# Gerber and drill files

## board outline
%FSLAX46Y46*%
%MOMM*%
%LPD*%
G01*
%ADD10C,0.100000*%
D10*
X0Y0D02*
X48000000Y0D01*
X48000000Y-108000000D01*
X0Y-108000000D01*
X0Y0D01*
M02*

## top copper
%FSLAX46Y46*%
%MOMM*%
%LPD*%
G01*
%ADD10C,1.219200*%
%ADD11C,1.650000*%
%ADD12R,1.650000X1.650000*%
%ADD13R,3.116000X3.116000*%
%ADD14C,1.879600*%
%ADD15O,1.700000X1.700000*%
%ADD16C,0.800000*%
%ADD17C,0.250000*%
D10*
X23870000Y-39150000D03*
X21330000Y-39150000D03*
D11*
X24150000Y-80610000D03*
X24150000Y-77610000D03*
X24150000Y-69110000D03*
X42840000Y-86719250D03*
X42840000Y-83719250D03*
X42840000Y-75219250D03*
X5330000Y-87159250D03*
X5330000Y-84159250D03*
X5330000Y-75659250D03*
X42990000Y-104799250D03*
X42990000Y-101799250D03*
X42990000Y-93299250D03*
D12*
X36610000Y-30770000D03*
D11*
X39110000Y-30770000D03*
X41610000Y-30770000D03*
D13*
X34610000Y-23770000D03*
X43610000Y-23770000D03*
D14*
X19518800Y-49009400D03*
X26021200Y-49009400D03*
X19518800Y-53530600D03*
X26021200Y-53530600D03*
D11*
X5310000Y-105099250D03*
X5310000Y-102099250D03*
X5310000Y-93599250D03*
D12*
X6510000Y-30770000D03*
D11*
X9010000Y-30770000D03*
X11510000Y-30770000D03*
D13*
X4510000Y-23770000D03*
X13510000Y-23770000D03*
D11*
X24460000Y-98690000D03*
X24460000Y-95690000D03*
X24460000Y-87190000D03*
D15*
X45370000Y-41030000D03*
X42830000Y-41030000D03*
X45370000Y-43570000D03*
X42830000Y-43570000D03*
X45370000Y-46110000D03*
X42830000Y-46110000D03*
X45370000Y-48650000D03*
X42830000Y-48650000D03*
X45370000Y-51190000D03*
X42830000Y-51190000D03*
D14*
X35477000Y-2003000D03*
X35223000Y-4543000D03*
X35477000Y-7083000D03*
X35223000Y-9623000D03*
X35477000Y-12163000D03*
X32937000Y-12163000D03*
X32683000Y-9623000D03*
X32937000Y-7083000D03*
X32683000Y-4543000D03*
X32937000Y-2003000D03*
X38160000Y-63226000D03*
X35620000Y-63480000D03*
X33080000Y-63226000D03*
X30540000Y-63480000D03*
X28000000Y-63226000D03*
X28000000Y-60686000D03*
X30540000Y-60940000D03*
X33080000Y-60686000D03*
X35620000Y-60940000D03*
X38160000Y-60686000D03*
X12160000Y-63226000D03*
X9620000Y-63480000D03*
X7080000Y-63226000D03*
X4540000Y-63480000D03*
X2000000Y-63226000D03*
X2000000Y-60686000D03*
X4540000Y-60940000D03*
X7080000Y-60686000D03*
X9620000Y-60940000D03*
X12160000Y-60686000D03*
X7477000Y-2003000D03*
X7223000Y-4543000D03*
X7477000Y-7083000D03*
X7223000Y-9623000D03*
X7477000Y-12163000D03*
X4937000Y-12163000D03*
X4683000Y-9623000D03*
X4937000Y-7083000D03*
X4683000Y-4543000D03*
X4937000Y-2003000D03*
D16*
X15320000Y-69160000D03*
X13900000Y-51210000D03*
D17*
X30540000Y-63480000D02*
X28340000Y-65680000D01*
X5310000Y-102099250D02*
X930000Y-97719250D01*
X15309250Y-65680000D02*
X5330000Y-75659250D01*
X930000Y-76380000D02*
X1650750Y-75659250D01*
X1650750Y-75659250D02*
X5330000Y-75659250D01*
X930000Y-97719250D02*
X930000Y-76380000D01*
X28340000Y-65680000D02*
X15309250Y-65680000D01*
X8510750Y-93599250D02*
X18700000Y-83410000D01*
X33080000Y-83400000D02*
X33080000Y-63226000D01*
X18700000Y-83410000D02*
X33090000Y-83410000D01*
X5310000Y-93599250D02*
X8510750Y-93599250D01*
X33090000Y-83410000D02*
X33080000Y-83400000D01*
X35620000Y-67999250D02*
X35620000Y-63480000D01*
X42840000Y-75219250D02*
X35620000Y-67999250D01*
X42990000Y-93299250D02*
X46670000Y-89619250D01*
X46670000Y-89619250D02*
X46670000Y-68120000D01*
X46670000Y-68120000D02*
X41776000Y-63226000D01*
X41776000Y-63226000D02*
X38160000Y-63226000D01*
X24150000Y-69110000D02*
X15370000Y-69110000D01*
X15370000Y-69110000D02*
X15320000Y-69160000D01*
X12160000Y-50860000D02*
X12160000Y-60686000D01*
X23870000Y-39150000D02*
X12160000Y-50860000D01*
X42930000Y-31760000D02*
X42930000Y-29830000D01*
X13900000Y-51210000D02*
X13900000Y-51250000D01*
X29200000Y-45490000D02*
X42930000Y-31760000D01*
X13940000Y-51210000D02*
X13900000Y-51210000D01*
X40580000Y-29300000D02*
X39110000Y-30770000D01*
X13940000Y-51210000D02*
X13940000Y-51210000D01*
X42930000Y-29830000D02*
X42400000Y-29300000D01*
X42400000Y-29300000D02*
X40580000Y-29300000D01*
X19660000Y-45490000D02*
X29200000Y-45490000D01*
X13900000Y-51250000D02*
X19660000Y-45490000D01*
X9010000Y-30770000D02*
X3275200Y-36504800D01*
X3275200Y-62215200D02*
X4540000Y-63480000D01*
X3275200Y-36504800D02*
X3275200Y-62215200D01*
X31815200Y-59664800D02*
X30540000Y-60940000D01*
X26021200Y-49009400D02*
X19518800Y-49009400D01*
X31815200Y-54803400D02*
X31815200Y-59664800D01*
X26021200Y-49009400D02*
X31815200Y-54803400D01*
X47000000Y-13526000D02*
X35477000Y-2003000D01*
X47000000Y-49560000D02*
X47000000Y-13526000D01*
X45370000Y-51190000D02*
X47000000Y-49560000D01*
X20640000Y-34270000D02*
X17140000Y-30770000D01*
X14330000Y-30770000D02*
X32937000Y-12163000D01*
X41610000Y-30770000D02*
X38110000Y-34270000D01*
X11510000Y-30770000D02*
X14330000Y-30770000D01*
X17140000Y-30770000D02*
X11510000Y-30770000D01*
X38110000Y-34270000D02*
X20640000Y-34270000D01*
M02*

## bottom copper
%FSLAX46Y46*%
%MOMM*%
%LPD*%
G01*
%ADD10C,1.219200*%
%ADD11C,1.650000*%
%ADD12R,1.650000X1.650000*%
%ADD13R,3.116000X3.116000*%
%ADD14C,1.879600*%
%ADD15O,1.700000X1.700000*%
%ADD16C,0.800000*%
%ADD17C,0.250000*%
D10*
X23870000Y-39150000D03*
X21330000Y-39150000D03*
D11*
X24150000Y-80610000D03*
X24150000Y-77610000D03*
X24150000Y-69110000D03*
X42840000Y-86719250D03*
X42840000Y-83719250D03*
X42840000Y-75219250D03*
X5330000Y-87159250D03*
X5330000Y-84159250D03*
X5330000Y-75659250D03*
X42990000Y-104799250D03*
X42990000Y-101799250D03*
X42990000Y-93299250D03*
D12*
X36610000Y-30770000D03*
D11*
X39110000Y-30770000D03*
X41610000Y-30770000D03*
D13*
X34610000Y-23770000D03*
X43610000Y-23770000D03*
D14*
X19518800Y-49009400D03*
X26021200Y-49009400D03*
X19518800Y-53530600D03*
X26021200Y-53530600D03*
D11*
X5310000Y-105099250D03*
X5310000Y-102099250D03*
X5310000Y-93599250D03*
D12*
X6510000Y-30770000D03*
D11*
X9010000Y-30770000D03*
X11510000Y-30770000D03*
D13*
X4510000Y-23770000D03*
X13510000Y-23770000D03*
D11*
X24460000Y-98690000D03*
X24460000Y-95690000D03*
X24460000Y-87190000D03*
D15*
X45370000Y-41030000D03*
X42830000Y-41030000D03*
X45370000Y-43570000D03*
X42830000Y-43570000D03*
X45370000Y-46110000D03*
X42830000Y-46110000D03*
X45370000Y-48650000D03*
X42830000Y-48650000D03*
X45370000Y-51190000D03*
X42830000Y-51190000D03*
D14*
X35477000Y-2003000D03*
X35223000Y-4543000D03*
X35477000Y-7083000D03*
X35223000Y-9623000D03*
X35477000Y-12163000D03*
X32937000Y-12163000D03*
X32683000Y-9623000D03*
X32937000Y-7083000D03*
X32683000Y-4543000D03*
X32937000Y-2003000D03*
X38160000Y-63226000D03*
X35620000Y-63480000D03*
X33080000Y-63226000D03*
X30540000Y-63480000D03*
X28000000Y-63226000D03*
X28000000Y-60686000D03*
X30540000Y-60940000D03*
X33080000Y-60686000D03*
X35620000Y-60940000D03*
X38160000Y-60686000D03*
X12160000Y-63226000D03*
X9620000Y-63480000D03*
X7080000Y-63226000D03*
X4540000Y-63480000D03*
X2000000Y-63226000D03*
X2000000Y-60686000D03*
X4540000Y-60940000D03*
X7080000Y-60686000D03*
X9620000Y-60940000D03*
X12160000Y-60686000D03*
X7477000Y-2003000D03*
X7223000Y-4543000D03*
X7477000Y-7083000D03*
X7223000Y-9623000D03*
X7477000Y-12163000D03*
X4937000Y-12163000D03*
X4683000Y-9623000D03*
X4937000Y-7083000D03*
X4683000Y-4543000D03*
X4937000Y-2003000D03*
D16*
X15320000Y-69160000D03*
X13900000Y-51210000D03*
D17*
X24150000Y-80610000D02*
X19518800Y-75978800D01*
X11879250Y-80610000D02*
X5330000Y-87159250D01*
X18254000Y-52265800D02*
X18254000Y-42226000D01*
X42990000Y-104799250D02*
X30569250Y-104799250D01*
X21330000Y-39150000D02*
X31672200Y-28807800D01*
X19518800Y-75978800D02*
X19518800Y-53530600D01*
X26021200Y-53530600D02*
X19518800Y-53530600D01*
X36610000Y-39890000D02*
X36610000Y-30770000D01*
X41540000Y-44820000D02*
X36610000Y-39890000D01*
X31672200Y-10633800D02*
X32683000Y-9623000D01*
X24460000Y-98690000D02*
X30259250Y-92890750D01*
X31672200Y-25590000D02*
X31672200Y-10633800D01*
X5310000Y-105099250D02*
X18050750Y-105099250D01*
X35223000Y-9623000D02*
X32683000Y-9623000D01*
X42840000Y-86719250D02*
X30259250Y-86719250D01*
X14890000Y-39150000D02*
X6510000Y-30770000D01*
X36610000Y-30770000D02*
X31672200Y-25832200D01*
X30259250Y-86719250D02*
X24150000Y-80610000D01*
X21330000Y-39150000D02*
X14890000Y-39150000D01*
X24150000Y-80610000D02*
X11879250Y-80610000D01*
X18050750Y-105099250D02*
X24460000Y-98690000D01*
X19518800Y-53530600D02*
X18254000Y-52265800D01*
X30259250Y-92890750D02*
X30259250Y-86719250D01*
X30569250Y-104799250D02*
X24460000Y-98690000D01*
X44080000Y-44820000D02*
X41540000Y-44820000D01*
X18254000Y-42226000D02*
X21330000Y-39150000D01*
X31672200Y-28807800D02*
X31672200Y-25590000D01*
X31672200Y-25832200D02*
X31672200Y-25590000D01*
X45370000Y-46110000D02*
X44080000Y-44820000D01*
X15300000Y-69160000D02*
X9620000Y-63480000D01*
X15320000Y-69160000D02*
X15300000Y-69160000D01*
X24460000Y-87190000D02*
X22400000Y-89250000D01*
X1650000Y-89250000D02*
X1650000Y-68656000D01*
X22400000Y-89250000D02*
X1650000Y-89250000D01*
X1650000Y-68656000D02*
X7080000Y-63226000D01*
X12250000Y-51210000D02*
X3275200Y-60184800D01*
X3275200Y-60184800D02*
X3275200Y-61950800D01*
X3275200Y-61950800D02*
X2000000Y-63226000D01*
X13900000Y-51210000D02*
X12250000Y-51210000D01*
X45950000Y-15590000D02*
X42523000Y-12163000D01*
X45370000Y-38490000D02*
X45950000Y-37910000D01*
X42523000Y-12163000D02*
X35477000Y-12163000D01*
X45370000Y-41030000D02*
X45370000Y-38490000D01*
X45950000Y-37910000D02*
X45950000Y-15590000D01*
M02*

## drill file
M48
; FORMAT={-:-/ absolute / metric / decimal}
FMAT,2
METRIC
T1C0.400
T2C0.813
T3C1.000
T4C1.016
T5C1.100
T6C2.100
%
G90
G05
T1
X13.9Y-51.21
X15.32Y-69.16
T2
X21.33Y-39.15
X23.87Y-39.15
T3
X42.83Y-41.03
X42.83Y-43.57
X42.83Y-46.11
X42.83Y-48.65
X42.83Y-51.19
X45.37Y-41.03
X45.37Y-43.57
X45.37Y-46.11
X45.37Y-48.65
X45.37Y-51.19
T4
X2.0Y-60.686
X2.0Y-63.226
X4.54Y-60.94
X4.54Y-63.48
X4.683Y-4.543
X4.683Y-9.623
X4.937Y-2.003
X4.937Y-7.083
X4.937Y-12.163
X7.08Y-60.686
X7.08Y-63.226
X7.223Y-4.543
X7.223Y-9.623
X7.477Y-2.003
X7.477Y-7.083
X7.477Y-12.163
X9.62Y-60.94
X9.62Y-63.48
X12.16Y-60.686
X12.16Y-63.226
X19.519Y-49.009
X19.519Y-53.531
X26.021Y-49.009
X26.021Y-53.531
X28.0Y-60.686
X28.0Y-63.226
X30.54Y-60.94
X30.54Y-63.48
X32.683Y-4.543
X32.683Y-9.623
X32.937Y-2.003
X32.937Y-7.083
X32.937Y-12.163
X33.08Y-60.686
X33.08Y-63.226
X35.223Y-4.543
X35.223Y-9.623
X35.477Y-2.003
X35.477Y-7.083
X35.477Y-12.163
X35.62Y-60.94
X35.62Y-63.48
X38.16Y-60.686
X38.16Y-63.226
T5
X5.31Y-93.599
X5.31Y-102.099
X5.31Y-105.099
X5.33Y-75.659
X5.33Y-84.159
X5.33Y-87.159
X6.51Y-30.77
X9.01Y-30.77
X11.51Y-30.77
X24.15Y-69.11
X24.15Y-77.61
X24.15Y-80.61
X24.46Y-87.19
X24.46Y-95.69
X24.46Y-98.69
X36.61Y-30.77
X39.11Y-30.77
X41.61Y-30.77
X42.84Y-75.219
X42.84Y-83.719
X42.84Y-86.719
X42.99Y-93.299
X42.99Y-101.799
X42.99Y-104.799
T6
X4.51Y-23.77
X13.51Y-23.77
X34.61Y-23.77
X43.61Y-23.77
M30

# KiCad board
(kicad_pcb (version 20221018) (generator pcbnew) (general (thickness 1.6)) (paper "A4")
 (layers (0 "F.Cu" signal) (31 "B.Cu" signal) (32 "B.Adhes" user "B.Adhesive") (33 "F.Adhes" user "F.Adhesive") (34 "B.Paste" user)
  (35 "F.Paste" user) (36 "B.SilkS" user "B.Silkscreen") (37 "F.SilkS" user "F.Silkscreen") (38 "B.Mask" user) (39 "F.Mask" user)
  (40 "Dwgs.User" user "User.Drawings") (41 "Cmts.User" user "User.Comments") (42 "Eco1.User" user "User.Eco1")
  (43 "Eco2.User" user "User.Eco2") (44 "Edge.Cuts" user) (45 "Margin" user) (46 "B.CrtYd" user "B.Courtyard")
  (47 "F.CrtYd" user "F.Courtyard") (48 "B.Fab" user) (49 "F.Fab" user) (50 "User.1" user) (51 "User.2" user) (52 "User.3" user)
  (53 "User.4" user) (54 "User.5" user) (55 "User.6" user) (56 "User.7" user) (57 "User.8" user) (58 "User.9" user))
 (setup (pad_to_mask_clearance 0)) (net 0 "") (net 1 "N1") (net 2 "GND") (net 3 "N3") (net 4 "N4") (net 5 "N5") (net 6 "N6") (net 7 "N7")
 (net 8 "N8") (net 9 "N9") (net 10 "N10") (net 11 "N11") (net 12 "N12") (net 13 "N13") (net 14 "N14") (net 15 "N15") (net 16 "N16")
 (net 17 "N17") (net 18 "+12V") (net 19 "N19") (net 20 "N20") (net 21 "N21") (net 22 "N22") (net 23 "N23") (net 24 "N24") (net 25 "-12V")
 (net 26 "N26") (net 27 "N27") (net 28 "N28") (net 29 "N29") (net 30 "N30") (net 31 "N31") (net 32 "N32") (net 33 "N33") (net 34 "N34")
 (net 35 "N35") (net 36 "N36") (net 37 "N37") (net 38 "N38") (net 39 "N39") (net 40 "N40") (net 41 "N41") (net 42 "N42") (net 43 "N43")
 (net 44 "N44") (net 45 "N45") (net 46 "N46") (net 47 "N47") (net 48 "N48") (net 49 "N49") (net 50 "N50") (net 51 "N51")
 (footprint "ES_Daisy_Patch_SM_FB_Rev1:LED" (layer "F.Cu") (at 22.6 39.15 180)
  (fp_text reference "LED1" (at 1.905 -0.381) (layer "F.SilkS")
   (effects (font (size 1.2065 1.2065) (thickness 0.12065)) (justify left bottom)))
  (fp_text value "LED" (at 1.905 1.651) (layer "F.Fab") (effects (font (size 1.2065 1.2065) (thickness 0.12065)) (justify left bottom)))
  (pad "A" thru_hole circle (at -1.27 0 180) (size 1.2192 1.2192) (drill 0.8128) (layers "*.Cu" "*.Mask") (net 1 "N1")
   (solder_mask_margin 0.0762))
  (pad "K" thru_hole circle (at 1.27 0 180) (size 1.2192 1.2192) (drill 0.8128) (layers "*.Cu" "*.Mask") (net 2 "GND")
   (solder_mask_margin 0.0762)))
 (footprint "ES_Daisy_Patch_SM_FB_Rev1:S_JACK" (layer "F.Cu") (at 24.15 74.11)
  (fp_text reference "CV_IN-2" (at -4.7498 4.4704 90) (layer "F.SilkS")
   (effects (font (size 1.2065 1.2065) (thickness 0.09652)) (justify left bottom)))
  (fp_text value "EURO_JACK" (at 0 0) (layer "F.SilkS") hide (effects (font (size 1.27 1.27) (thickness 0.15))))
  (pad "GND" thru_hole circle (at 0 6.5) (size 1.65 1.65) (drill 1.1) (layers "*.Cu" "*.Mask") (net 2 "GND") (solder_mask_margin 0.0762))
  (pad "NORM" thru_hole circle (at 0 3.5) (size 1.65 1.65) (drill 1.1) (layers "*.Cu" "*.Mask") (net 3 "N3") (solder_mask_margin 0.0762))
  (pad "TIP" thru_hole circle (at 0 -5) (size 1.65 1.65) (drill 1.1) (layers "*.Cu" "*.Mask") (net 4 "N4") (solder_mask_margin 0.0762)
   (zone_connect 2)))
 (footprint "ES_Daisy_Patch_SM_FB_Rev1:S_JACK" (layer "F.Cu") (at 42.84 80.21925)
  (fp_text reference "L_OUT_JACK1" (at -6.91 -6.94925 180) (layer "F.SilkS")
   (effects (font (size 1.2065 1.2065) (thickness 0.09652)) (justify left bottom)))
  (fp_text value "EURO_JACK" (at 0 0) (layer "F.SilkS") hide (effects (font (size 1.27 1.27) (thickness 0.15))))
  (pad "GND" thru_hole circle (at 0 6.5) (size 1.65 1.65) (drill 1.1) (layers "*.Cu" "*.Mask") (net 2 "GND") (solder_mask_margin 0.0762))
  (pad "NORM" thru_hole circle (at 0 3.5) (size 1.65 1.65) (drill 1.1) (layers "*.Cu" "*.Mask") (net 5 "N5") (solder_mask_margin 0.0762))
  (pad "TIP" thru_hole circle (at 0 -5) (size 1.65 1.65) (drill 1.1) (layers "*.Cu" "*.Mask") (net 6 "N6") (solder_mask_margin 0.0762)
   (zone_connect 2)))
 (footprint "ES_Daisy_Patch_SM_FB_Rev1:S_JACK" (layer "F.Cu") (at 5.33 80.65925)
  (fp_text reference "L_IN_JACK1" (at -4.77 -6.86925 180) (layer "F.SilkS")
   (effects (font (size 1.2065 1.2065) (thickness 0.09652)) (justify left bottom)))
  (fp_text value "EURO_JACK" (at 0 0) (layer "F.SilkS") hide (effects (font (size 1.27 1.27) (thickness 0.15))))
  (pad "GND" thru_hole circle (at 0 6.5) (size 1.65 1.65) (drill 1.1) (layers "*.Cu" "*.Mask") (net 2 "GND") (solder_mask_margin 0.0762))
  (pad "NORM" thru_hole circle (at 0 3.5) (size 1.65 1.65) (drill 1.1) (layers "*.Cu" "*.Mask") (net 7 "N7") (solder_mask_margin 0.0762))
  (pad "TIP" thru_hole circle (at 0 -5) (size 1.65 1.65) (drill 1.1) (layers "*.Cu" "*.Mask") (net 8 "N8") (solder_mask_margin 0.0762)
   (zone_connect 2)))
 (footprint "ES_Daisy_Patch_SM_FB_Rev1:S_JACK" (layer "F.Cu") (at 42.99 98.29925)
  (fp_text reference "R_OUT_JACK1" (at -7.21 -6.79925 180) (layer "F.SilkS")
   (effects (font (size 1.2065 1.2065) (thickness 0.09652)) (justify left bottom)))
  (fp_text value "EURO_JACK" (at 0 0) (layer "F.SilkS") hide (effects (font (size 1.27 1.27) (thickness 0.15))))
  (pad "GND" thru_hole circle (at 0 6.5) (size 1.65 1.65) (drill 1.1) (layers "*.Cu" "*.Mask") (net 2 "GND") (solder_mask_margin 0.0762))
  (pad "NORM" thru_hole circle (at 0 3.5) (size 1.65 1.65) (drill 1.1) (layers "*.Cu" "*.Mask") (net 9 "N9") (solder_mask_margin 0.0762))
  (pad "TIP" thru_hole circle (at 0 -5) (size 1.65 1.65) (drill 1.1) (layers "*.Cu" "*.Mask") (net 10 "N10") (solder_mask_margin 0.0762)
   (zone_connect 2)))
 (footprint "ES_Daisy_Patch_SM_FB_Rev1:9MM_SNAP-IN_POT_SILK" (layer "F.Cu") (at 39.11 23.77)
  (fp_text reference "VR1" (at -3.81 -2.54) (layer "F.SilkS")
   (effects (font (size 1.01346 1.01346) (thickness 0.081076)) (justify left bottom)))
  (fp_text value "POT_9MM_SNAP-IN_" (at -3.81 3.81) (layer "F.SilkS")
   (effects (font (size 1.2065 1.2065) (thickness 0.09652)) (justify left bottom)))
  (pad "1" thru_hole rect (at -2.5 7 270) (size 1.65 1.65) (drill 1.1) (layers "*.Cu" "*.Mask") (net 2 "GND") (solder_mask_margin 0.0762))
  (pad "2" thru_hole circle (at 0 7 270) (size 1.65 1.65) (drill 1.1) (layers "*.Cu" "*.Mask") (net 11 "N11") (solder_mask_margin 0.0762))
  (pad "3" thru_hole circle (at 2.5 7 270) (size 1.65 1.65) (drill 1.1) (layers "*.Cu" "*.Mask") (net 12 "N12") (solder_mask_margin 0.0762))
  (pad "CHASSIS1" thru_hole rect (at -4.5 0 270) (size 3.116 3.116) (drill 2.1) (layers "*.Cu" "*.Mask") (solder_mask_margin 0.0762))
  (pad "CHASSIS2" thru_hole rect (at 4.5 0 270) (size 3.116 3.116) (drill 2.1) (layers "*.Cu" "*.Mask") (solder_mask_margin 0.0762)))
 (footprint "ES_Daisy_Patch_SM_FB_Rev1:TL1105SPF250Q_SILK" (layer "F.Cu") (at 22.77 51.27)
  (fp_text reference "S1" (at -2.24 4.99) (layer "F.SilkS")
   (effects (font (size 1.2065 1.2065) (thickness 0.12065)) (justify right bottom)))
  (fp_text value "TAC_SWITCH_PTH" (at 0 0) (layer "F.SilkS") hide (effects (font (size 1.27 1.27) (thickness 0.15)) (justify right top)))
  (pad "1" thru_hole circle (at -3.2512 -2.2606) (size 1.8796 1.8796) (drill 1.016) (layers "*.Cu" "*.Mask") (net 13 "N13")
   (solder_mask_margin 0.0762))
  (pad "2" thru_hole circle (at 3.2512 -2.2606) (size 1.8796 1.8796) (drill 1.016) (layers "*.Cu" "*.Mask") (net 13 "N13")
   (solder_mask_margin 0.0762))
  (pad "3" thru_hole circle (at -3.2512 2.2606) (size 1.8796 1.8796) (drill 1.016) (layers "*.Cu" "*.Mask") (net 2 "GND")
   (solder_mask_margin 0.0762))
  (pad "4" thru_hole circle (at 3.2512 2.2606) (size 1.8796 1.8796) (drill 1.016) (layers "*.Cu" "*.Mask") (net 2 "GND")
   (solder_mask_margin 0.0762)))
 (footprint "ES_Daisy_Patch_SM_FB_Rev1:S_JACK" (layer "F.Cu") (at 5.31 98.59925)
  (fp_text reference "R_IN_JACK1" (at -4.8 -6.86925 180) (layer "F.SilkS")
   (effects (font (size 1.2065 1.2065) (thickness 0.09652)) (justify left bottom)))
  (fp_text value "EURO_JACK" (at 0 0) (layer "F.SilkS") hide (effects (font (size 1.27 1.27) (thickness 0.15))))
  (pad "GND" thru_hole circle (at 0 6.5) (size 1.65 1.65) (drill 1.1) (layers "*.Cu" "*.Mask") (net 2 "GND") (solder_mask_margin 0.0762))
  (pad "NORM" thru_hole circle (at 0 3.5) (size 1.65 1.65) (drill 1.1) (layers "*.Cu" "*.Mask") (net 8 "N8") (solder_mask_margin 0.0762))
  (pad "TIP" thru_hole circle (at 0 -5) (size 1.65 1.65) (drill 1.1) (layers "*.Cu" "*.Mask") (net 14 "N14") (solder_mask_margin 0.0762)
   (zone_connect 2)))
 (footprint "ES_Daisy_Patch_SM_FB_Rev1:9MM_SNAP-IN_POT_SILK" (layer "F.Cu") (at 9.01 23.77)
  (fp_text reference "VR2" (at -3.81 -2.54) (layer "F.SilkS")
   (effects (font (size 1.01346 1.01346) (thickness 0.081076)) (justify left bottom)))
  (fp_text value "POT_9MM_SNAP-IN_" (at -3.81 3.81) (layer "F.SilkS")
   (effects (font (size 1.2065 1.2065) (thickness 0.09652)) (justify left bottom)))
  (pad "1" thru_hole rect (at -2.5 7 270) (size 1.65 1.65) (drill 1.1) (layers "*.Cu" "*.Mask") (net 2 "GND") (solder_mask_margin 0.0762))
  (pad "2" thru_hole circle (at 0 7 270) (size 1.65 1.65) (drill 1.1) (layers "*.Cu" "*.Mask") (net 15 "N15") (solder_mask_margin 0.0762))
  (pad "3" thru_hole circle (at 2.5 7 270) (size 1.65 1.65) (drill 1.1) (layers "*.Cu" "*.Mask") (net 12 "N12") (solder_mask_margin 0.0762))
  (pad "CHASSIS1" thru_hole rect (at -4.5 0 270) (size 3.116 3.116) (drill 2.1) (layers "*.Cu" "*.Mask") (solder_mask_margin 0.0762))
  (pad "CHASSIS2" thru_hole rect (at 4.5 0 270) (size 3.116 3.116) (drill 2.1) (layers "*.Cu" "*.Mask") (solder_mask_margin 0.0762)))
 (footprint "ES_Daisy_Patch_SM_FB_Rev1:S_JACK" (layer "F.Cu") (at 24.46 92.19)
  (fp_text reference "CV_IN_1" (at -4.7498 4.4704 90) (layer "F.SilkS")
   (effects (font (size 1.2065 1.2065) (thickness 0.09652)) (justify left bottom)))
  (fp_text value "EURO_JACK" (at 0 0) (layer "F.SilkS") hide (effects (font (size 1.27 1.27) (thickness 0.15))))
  (pad "GND" thru_hole circle (at 0 6.5) (size 1.65 1.65) (drill 1.1) (layers "*.Cu" "*.Mask") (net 2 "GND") (solder_mask_margin 0.0762))
  (pad "NORM" thru_hole circle (at 0 3.5) (size 1.65 1.65) (drill 1.1) (layers "*.Cu" "*.Mask") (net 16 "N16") (solder_mask_margin 0.0762))
  (pad "TIP" thru_hole circle (at 0 -5) (size 1.65 1.65) (drill 1.1) (layers "*.Cu" "*.Mask") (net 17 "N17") (solder_mask_margin 0.0762)
   (zone_connect 2)))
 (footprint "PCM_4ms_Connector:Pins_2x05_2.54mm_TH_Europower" (layer "B.Cu") (at 44.1 46.11 180)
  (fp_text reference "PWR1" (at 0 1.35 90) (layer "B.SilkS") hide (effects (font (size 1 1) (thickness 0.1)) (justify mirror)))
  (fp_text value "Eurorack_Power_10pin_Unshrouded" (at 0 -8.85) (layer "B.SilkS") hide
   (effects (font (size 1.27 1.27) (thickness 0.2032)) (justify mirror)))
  (pad "1" thru_hole oval (at -1.27 5.08 180) (size 1.7 1.7) (drill 1) (layers "*.Cu" "*.Mask") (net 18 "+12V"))
  (pad "2" thru_hole oval (at 1.27 5.08 180) (size 1.7 1.7) (drill 1) (layers "*.Cu" "*.Mask") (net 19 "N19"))
  (pad "3" thru_hole oval (at -1.27 2.54 180) (size 1.7 1.7) (drill 1) (layers "*.Cu" "*.Mask") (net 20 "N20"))
  (pad "4" thru_hole oval (at 1.27 2.54 180) (size 1.7 1.7) (drill 1) (layers "*.Cu" "*.Mask") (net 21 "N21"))
  (pad "5" thru_hole oval (at -1.27 0 180) (size 1.7 1.7) (drill 1) (layers "*.Cu" "*.Mask") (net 2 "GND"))
  (pad "6" thru_hole oval (at 1.27 0 180) (size 1.7 1.7) (drill 1) (layers "*.Cu" "*.Mask") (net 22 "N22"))
  (pad "7" thru_hole oval (at -1.27 -2.54 180) (size 1.7 1.7) (drill 1) (layers "*.Cu" "*.Mask") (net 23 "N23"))
  (pad "8" thru_hole oval (at 1.27 -2.54 180) (size 1.7 1.7) (drill 1) (layers "*.Cu" "*.Mask") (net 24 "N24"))
  (pad "9" thru_hole oval (at -1.27 -5.08 180) (size 1.7 1.7) (drill 1) (layers "*.Cu" "*.Mask") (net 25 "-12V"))
  (pad "10" thru_hole oval (at 1.27 -5.08 180) (size 1.7 1.7) (drill 1) (layers "*.Cu" "*.Mask") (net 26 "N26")))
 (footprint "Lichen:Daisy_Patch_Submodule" (layer "B.Cu") (at 20.08 34.083 -90)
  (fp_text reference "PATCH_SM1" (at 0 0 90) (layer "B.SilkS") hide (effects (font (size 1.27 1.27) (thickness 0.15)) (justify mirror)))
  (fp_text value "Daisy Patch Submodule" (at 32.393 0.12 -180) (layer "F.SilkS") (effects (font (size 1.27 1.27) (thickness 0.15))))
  (pad "A1" thru_hole circle (at -32.08 -15.397) (size 1.8796 1.8796) (drill 1.016) (layers "*.Cu" "*.Mask") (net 25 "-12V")
   (solder_mask_margin 0.0762))
  (pad "A2" thru_hole circle (at -29.54 -15.143) (size 1.8796 1.8796) (drill 1.016) (layers "*.Cu" "*.Mask") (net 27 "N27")
   (solder_mask_margin 0.0762))
  (pad "A3" thru_hole circle (at -27 -15.397) (size 1.8796 1.8796) (drill 1.016) (layers "*.Cu" "*.Mask") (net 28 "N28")
   (solder_mask_margin 0.0762))
  (pad "A4" thru_hole circle (at -24.46 -15.143) (size 1.8796 1.8796) (drill 1.016) (layers "*.Cu" "*.Mask") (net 2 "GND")
   (solder_mask_margin 0.0762))
  (pad "A5" thru_hole circle (at -21.92 -15.397) (size 1.8796 1.8796) (drill 1.016) (layers "*.Cu" "*.Mask") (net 18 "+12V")
   (solder_mask_margin 0.0762))
  (pad "A6" thru_hole circle (at -21.92 -12.857) (size 1.8796 1.8796) (drill 1.016) (layers "*.Cu" "*.Mask") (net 12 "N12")
   (solder_mask_margin 0.0762))
  (pad "A7" thru_hole circle (at -24.46 -12.603) (size 1.8796 1.8796) (drill 1.016) (layers "*.Cu" "*.Mask") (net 2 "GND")
   (solder_mask_margin 0.0762))
  (pad "A8" thru_hole circle (at -27 -12.857) (size 1.8796 1.8796) (drill 1.016) (layers "*.Cu" "*.Mask") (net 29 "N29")
   (solder_mask_margin 0.0762))
  (pad "A9" thru_hole circle (at -29.54 -12.603) (size 1.8796 1.8796) (drill 1.016) (layers "*.Cu" "*.Mask") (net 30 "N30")
   (solder_mask_margin 0.0762))
  (pad "A10" thru_hole circle (at -32.08 -12.857) (size 1.8796 1.8796) (drill 1.016) (layers "*.Cu" "*.Mask") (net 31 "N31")
   (solder_mask_margin 0.0762))
  (pad "B1" thru_hole circle (at 29.143 -18.08 90) (size 1.8796 1.8796) (drill 1.016) (layers "*.Cu" "*.Mask") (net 10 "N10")
   (solder_mask_margin 0.0762))
  (pad "B2" thru_hole circle (at 29.397 -15.54 90) (size 1.8796 1.8796) (drill 1.016) (layers "*.Cu" "*.Mask") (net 6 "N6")
   (solder_mask_margin 0.0762))
  (pad "B3" thru_hole circle (at 29.143 -13 90) (size 1.8796 1.8796) (drill 1.016) (layers "*.Cu" "*.Mask") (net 14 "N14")
   (solder_mask_margin 0.0762))
  (pad "B4" thru_hole circle (at 29.397 -10.46 90) (size 1.8796 1.8796) (drill 1.016) (layers "*.Cu" "*.Mask") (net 8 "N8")
   (solder_mask_margin 0.0762))
  (pad "B5" thru_hole circle (at 29.143 -7.92 90) (size 1.8796 1.8796) (drill 1.016) (layers "*.Cu" "*.Mask") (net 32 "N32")
   (solder_mask_margin 0.0762))
  (pad "B6" thru_hole circle (at 26.603 -7.92 90) (size 1.8796 1.8796) (drill 1.016) (layers "*.Cu" "*.Mask") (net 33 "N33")
   (solder_mask_margin 0.0762))
  (pad "B7" thru_hole circle (at 26.857 -10.46 90) (size 1.8796 1.8796) (drill 1.016) (layers "*.Cu" "*.Mask") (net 13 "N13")
   (solder_mask_margin 0.0762))
  (pad "B8" thru_hole circle (at 26.603 -13 90) (size 1.8796 1.8796) (drill 1.016) (layers "*.Cu" "*.Mask") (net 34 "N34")
   (solder_mask_margin 0.0762))
  (pad "B9" thru_hole circle (at 26.857 -15.54 90) (size 1.8796 1.8796) (drill 1.016) (layers "*.Cu" "*.Mask") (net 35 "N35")
   (solder_mask_margin 0.0762))
  (pad "B10" thru_hole circle (at 26.603 -18.08 90) (size 1.8796 1.8796) (drill 1.016) (layers "*.Cu" "*.Mask") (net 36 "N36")
   (solder_mask_margin 0.0762))
  (pad "C1" thru_hole circle (at 29.143 7.92 90) (size 1.8796 1.8796) (drill 1.016) (layers "*.Cu" "*.Mask") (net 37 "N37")
   (solder_mask_margin 0.0762))
  (pad "C2" thru_hole circle (at 29.397 10.46 90) (size 1.8796 1.8796) (drill 1.016) (layers "*.Cu" "*.Mask") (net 4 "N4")
   (solder_mask_margin 0.0762))
  (pad "C3" thru_hole circle (at 29.143 13 90) (size 1.8796 1.8796) (drill 1.016) (layers "*.Cu" "*.Mask") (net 17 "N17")
   (solder_mask_margin 0.0762))
  (pad "C4" thru_hole circle (at 29.397 15.54 90) (size 1.8796 1.8796) (drill 1.016) (layers "*.Cu" "*.Mask") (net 15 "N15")
   (solder_mask_margin 0.0762))
  (pad "C5" thru_hole circle (at 29.143 18.08 90) (size 1.8796 1.8796) (drill 1.016) (layers "*.Cu" "*.Mask") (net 11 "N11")
   (solder_mask_margin 0.0762))
  (pad "C6" thru_hole circle (at 26.603 18.08 90) (size 1.8796 1.8796) (drill 1.016) (layers "*.Cu" "*.Mask") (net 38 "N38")
   (solder_mask_margin 0.0762))
  (pad "C7" thru_hole circle (at 26.857 15.54 90) (size 1.8796 1.8796) (drill 1.016) (layers "*.Cu" "*.Mask") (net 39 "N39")
   (solder_mask_margin 0.0762))
  (pad "C8" thru_hole circle (at 26.603 13 90) (size 1.8796 1.8796) (drill 1.016) (layers "*.Cu" "*.Mask") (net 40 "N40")
   (solder_mask_margin 0.0762))
  (pad "C9" thru_hole circle (at 26.857 10.46 90) (size 1.8796 1.8796) (drill 1.016) (layers "*.Cu" "*.Mask") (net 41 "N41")
   (solder_mask_margin 0.0762))
  (pad "C10" thru_hole circle (at 26.603 7.92 90) (size 1.8796 1.8796) (drill 1.016) (layers "*.Cu" "*.Mask") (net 1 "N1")
   (solder_mask_margin 0.0762))
  (pad "D1" thru_hole circle (at -32.08 12.603) (size 1.8796 1.8796) (drill 1.016) (layers "*.Cu" "*.Mask") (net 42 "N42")
   (solder_mask_margin 0.0762))
  (pad "D2" thru_hole circle (at -29.54 12.857) (size 1.8796 1.8796) (drill 1.016) (layers "*.Cu" "*.Mask") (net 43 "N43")
   (solder_mask_margin 0.0762))
  (pad "D3" thru_hole circle (at -27 12.603) (size 1.8796 1.8796) (drill 1.016) (layers "*.Cu" "*.Mask") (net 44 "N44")
   (solder_mask_margin 0.0762))
  (pad "D4" thru_hole circle (at -24.46 12.857) (size 1.8796 1.8796) (drill 1.016) (layers "*.Cu" "*.Mask") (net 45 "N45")
   (solder_mask_margin 0.0762))
  (pad "D5" thru_hole circle (at -21.92 12.603) (size 1.8796 1.8796) (drill 1.016) (layers "*.Cu" "*.Mask") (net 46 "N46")
   (solder_mask_margin 0.0762))
  (pad "D6" thru_hole circle (at -21.92 15.143) (size 1.8796 1.8796) (drill 1.016) (layers "*.Cu" "*.Mask") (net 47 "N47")
   (solder_mask_margin 0.0762))
  (pad "D7" thru_hole circle (at -24.46 15.397) (size 1.8796 1.8796) (drill 1.016) (layers "*.Cu" "*.Mask") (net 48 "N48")
   (solder_mask_margin 0.0762))
  (pad "D8" thru_hole circle (at -27 15.143) (size 1.8796 1.8796) (drill 1.016) (layers "*.Cu" "*.Mask") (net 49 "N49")
   (solder_mask_margin 0.0762))
  (pad "D9" thru_hole circle (at -29.54 15.397) (size 1.8796 1.8796) (drill 1.016) (layers "*.Cu" "*.Mask") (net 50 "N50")
   (solder_mask_margin 0.0762))
  (pad "D10" thru_hole circle (at -32.08 15.143) (size 1.8796 1.8796) (drill 1.016) (layers "*.Cu" "*.Mask") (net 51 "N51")
   (solder_mask_margin 0.0762)))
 (gr_rect (start 0 0) (end 48 108) (stroke (width 0.1) (type default)) (fill none) (layer "Edge.Cuts"))
 (segment (start 30.54 63.48) (end 28.34 65.68) (width 0.25) (layer "F.Cu") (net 8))
 (segment (start 5.31 102.09925) (end 0.93 97.71925) (width 0.25) (layer "F.Cu") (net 8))
 (segment (start 15.30925 65.68) (end 5.33 75.65925) (width 0.25) (layer "F.Cu") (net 8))
 (segment (start 0.93 76.38) (end 1.65075 75.65925) (width 0.25) (layer "F.Cu") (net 8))
 (segment (start 1.65075 75.65925) (end 5.33 75.65925) (width 0.25) (layer "F.Cu") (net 8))
 (segment (start 0.93 97.71925) (end 0.93 76.38) (width 0.25) (layer "F.Cu") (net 8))
 (segment (start 28.34 65.68) (end 15.30925 65.68) (width 0.25) (layer "F.Cu") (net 8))
 (segment (start 8.51075 93.59925) (end 18.7 83.41) (width 0.25) (layer "F.Cu") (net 14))
 (segment (start 33.08 83.4) (end 33.08 63.226) (width 0.25) (layer "F.Cu") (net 14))
 (segment (start 18.7 83.41) (end 33.09 83.41) (width 0.25) (layer "F.Cu") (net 14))
 (segment (start 5.31 93.59925) (end 8.51075 93.59925) (width 0.25) (layer "F.Cu") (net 14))
 (segment (start 33.09 83.41) (end 33.08 83.4) (width 0.25) (layer "F.Cu") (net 14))
 (segment (start 24.15 80.61) (end 19.5188 75.9788) (width 0.25) (layer "B.Cu") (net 2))
 (segment (start 11.87925 80.61) (end 5.33 87.15925) (width 0.25) (layer "B.Cu") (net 2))
 (segment (start 18.254 52.2658) (end 18.254 42.226) (width 0.25) (layer "B.Cu") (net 2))
 (segment (start 42.99 104.79925) (end 30.56925 104.79925) (width 0.25) (layer "B.Cu") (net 2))
 (segment (start 21.33 39.15) (end 31.6722 28.8078) (width 0.25) (layer "B.Cu") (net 2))
 (segment (start 19.5188 75.9788) (end 19.5188 53.5306) (width 0.25) (layer "B.Cu") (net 2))
 (segment (start 26.0212 53.5306) (end 19.5188 53.5306) (width 0.25) (layer "B.Cu") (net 2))
 (segment (start 36.61 39.89) (end 36.61 30.77) (width 0.25) (layer "B.Cu") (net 2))
 (segment (start 41.54 44.82) (end 36.61 39.89) (width 0.25) (layer "B.Cu") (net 2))
 (segment (start 31.6722 10.6338) (end 32.683 9.623) (width 0.25) (layer "B.Cu") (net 2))
 (segment (start 24.46 98.69) (end 30.25925 92.89075) (width 0.25) (layer "B.Cu") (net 2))
 (segment (start 31.6722 25.59) (end 31.6722 10.6338) (width 0.25) (layer "B.Cu") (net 2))
 (segment (start 5.31 105.09925) (end 18.05075 105.09925) (width 0.25) (layer "B.Cu") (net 2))
 (segment (start 35.223 9.623) (end 32.683 9.623) (width 0.25) (layer "B.Cu") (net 2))
 (segment (start 42.84 86.71925) (end 30.25925 86.71925) (width 0.25) (layer "B.Cu") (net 2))
 (segment (start 14.89 39.15) (end 6.51 30.77) (width 0.25) (layer "B.Cu") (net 2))
 (segment (start 36.61 30.77) (end 31.6722 25.8322) (width 0.25) (layer "B.Cu") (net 2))
 (segment (start 30.25925 86.71925) (end 24.15 80.61) (width 0.25) (layer "B.Cu") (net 2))
 (segment (start 21.33 39.15) (end 14.89 39.15) (width 0.25) (layer "B.Cu") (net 2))
 (segment (start 24.15 80.61) (end 11.87925 80.61) (width 0.25) (layer "B.Cu") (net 2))
 (segment (start 18.05075 105.09925) (end 24.46 98.69) (width 0.25) (layer "B.Cu") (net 2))
 (segment (start 19.5188 53.5306) (end 18.254 52.2658) (width 0.25) (layer "B.Cu") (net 2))
 (segment (start 30.25925 92.89075) (end 30.25925 86.71925) (width 0.25) (layer "B.Cu") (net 2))
 (segment (start 30.56925 104.79925) (end 24.46 98.69) (width 0.25) (layer "B.Cu") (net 2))
 (segment (start 44.08 44.82) (end 41.54 44.82) (width 0.25) (layer "B.Cu") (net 2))
 (segment (start 18.254 42.226) (end 21.33 39.15) (width 0.25) (layer "B.Cu") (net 2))
 (segment (start 31.6722 28.8078) (end 31.6722 25.59) (width 0.25) (layer "B.Cu") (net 2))
 (segment (start 31.6722 25.8322) (end 31.6722 25.59) (width 0.25) (layer "B.Cu") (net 2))
 (segment (start 45.37 46.11) (end 44.08 44.82) (width 0.25) (layer "B.Cu") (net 2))
 (segment (start 35.62 67.99925) (end 35.62 63.48) (width 0.25) (layer "F.Cu") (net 6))
 (segment (start 42.84 75.21925) (end 35.62 67.99925) (width 0.25) (layer "F.Cu") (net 6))
 (segment (start 42.99 93.29925) (end 46.67 89.61925) (width 0.25) (layer "F.Cu") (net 10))
 (segment (start 46.67 89.61925) (end 46.67 68.12) (width 0.25) (layer "F.Cu") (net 10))
 (segment (start 46.67 68.12) (end 41.776 63.226) (width 0.25) (layer "F.Cu") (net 10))
 (segment (start 41.776 63.226) (end 38.16 63.226) (width 0.25) (layer "F.Cu") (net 10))
 (segment (start 24.15 69.11) (end 15.37 69.11) (width 0.25) (layer "F.Cu") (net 4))
 (segment (start 15.37 69.11) (end 15.32 69.16) (width 0.25) (layer "F.Cu") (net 4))
 (via (at 15.32 69.16) (size 0.8) (drill 0.4) (layers "F.Cu" "B.Cu") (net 4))
 (segment (start 15.3 69.16) (end 9.62 63.48) (width 0.25) (layer "B.Cu") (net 4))
 (segment (start 15.32 69.16) (end 15.3 69.16) (width 0.25) (layer "B.Cu") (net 4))
 (segment (start 24.46 87.19) (end 22.4 89.25) (width 0.25) (layer "B.Cu") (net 17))
 (segment (start 1.65 89.25) (end 1.65 68.656) (width 0.25) (layer "B.Cu") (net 17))
 (segment (start 22.4 89.25) (end 1.65 89.25) (width 0.25) (layer "B.Cu") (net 17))
 (segment (start 1.65 68.656) (end 7.08 63.226) (width 0.25) (layer "B.Cu") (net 17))
 (segment (start 12.16 50.86) (end 12.16 60.686) (width 0.25) (layer "F.Cu") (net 1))
 (segment (start 23.87 39.15) (end 12.16 50.86) (width 0.25) (layer "F.Cu") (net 1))
 (segment (start 42.93 31.76) (end 42.93 29.83) (width 0.25) (layer "F.Cu") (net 11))
 (segment (start 13.9 51.21) (end 13.9 51.25) (width 0.25) (layer "F.Cu") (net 11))
 (segment (start 29.2 45.49) (end 42.93 31.76) (width 0.25) (layer "F.Cu") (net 11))
 (segment (start 13.94 51.21) (end 13.9 51.21) (width 0.25) (layer "F.Cu") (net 11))
 (segment (start 40.58 29.3) (end 39.11 30.77) (width 0.25) (layer "F.Cu") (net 11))
 (segment (start 13.94 51.21) (end 13.94 51.21) (width 0.25) (layer "F.Cu") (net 11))
 (segment (start 42.93 29.83) (end 42.4 29.3) (width 0.25) (layer "F.Cu") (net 11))
 (segment (start 42.4 29.3) (end 40.58 29.3) (width 0.25) (layer "F.Cu") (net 11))
 (segment (start 19.66 45.49) (end 29.2 45.49) (width 0.25) (layer "F.Cu") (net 11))
 (segment (start 13.9 51.25) (end 19.66 45.49) (width 0.25) (layer "F.Cu") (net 11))
 (via (at 13.9 51.21) (size 0.8) (drill 0.4) (layers "F.Cu" "B.Cu") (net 11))
 (segment (start 12.25 51.21) (end 3.2752 60.1848) (width 0.25) (layer "B.Cu") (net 11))
 (segment (start 3.2752 60.1848) (end 3.2752 61.9508) (width 0.25) (layer "B.Cu") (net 11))
 (segment (start 3.2752 61.9508) (end 2 63.226) (width 0.25) (layer "B.Cu") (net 11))
 (segment (start 13.9 51.21) (end 12.25 51.21) (width 0.25) (layer "B.Cu") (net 11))
 (segment (start 9.01 30.77) (end 3.2752 36.5048) (width 0.25) (layer "F.Cu") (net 15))
 (segment (start 3.2752 62.2152) (end 4.54 63.48) (width 0.25) (layer "F.Cu") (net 15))
 (segment (start 3.2752 36.5048) (end 3.2752 62.2152) (width 0.25) (layer "F.Cu") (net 15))
 (segment (start 31.8152 59.6648) (end 30.54 60.94) (width 0.25) (layer "F.Cu") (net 13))
 (segment (start 26.0212 49.0094) (end 19.5188 49.0094) (width 0.25) (layer "F.Cu") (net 13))
 (segment (start 31.8152 54.8034) (end 31.8152 59.6648) (width 0.25) (layer "F.Cu") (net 13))
 (segment (start 26.0212 49.0094) (end 31.8152 54.8034) (width 0.25) (layer "F.Cu") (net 13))
 (segment (start 47 13.526) (end 35.477 2.003) (width 0.25) (layer "F.Cu") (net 25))
 (segment (start 47 49.56) (end 47 13.526) (width 0.25) (layer "F.Cu") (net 25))
 (segment (start 45.37 51.19) (end 47 49.56) (width 0.25) (layer "F.Cu") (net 25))
 (segment (start 45.95 15.59) (end 42.523 12.163) (width 0.25) (layer "B.Cu") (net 18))
 (segment (start 45.37 38.49) (end 45.95 37.91) (width 0.25) (layer "B.Cu") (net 18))
 (segment (start 42.523 12.163) (end 35.477 12.163) (width 0.25) (layer "B.Cu") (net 18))
 (segment (start 45.37 41.03) (end 45.37 38.49) (width 0.25) (layer "B.Cu") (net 18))
 (segment (start 45.95 37.91) (end 45.95 15.59) (width 0.25) (layer "B.Cu") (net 18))
 (segment (start 20.64 34.27) (end 17.14 30.77) (width 0.25) (layer "F.Cu") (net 12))
 (segment (start 14.33 30.77) (end 32.937 12.163) (width 0.25) (layer "F.Cu") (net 12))
 (segment (start 41.61 30.77) (end 38.11 34.27) (width 0.25) (layer "F.Cu") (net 12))
 (segment (start 11.51 30.77) (end 14.33 30.77) (width 0.25) (layer "F.Cu") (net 12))
 (segment (start 17.14 30.77) (end 11.51 30.77) (width 0.25) (layer "F.Cu") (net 12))
 (segment (start 38.11 34.27) (end 20.64 34.27) (width 0.25) (layer "F.Cu") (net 12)))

